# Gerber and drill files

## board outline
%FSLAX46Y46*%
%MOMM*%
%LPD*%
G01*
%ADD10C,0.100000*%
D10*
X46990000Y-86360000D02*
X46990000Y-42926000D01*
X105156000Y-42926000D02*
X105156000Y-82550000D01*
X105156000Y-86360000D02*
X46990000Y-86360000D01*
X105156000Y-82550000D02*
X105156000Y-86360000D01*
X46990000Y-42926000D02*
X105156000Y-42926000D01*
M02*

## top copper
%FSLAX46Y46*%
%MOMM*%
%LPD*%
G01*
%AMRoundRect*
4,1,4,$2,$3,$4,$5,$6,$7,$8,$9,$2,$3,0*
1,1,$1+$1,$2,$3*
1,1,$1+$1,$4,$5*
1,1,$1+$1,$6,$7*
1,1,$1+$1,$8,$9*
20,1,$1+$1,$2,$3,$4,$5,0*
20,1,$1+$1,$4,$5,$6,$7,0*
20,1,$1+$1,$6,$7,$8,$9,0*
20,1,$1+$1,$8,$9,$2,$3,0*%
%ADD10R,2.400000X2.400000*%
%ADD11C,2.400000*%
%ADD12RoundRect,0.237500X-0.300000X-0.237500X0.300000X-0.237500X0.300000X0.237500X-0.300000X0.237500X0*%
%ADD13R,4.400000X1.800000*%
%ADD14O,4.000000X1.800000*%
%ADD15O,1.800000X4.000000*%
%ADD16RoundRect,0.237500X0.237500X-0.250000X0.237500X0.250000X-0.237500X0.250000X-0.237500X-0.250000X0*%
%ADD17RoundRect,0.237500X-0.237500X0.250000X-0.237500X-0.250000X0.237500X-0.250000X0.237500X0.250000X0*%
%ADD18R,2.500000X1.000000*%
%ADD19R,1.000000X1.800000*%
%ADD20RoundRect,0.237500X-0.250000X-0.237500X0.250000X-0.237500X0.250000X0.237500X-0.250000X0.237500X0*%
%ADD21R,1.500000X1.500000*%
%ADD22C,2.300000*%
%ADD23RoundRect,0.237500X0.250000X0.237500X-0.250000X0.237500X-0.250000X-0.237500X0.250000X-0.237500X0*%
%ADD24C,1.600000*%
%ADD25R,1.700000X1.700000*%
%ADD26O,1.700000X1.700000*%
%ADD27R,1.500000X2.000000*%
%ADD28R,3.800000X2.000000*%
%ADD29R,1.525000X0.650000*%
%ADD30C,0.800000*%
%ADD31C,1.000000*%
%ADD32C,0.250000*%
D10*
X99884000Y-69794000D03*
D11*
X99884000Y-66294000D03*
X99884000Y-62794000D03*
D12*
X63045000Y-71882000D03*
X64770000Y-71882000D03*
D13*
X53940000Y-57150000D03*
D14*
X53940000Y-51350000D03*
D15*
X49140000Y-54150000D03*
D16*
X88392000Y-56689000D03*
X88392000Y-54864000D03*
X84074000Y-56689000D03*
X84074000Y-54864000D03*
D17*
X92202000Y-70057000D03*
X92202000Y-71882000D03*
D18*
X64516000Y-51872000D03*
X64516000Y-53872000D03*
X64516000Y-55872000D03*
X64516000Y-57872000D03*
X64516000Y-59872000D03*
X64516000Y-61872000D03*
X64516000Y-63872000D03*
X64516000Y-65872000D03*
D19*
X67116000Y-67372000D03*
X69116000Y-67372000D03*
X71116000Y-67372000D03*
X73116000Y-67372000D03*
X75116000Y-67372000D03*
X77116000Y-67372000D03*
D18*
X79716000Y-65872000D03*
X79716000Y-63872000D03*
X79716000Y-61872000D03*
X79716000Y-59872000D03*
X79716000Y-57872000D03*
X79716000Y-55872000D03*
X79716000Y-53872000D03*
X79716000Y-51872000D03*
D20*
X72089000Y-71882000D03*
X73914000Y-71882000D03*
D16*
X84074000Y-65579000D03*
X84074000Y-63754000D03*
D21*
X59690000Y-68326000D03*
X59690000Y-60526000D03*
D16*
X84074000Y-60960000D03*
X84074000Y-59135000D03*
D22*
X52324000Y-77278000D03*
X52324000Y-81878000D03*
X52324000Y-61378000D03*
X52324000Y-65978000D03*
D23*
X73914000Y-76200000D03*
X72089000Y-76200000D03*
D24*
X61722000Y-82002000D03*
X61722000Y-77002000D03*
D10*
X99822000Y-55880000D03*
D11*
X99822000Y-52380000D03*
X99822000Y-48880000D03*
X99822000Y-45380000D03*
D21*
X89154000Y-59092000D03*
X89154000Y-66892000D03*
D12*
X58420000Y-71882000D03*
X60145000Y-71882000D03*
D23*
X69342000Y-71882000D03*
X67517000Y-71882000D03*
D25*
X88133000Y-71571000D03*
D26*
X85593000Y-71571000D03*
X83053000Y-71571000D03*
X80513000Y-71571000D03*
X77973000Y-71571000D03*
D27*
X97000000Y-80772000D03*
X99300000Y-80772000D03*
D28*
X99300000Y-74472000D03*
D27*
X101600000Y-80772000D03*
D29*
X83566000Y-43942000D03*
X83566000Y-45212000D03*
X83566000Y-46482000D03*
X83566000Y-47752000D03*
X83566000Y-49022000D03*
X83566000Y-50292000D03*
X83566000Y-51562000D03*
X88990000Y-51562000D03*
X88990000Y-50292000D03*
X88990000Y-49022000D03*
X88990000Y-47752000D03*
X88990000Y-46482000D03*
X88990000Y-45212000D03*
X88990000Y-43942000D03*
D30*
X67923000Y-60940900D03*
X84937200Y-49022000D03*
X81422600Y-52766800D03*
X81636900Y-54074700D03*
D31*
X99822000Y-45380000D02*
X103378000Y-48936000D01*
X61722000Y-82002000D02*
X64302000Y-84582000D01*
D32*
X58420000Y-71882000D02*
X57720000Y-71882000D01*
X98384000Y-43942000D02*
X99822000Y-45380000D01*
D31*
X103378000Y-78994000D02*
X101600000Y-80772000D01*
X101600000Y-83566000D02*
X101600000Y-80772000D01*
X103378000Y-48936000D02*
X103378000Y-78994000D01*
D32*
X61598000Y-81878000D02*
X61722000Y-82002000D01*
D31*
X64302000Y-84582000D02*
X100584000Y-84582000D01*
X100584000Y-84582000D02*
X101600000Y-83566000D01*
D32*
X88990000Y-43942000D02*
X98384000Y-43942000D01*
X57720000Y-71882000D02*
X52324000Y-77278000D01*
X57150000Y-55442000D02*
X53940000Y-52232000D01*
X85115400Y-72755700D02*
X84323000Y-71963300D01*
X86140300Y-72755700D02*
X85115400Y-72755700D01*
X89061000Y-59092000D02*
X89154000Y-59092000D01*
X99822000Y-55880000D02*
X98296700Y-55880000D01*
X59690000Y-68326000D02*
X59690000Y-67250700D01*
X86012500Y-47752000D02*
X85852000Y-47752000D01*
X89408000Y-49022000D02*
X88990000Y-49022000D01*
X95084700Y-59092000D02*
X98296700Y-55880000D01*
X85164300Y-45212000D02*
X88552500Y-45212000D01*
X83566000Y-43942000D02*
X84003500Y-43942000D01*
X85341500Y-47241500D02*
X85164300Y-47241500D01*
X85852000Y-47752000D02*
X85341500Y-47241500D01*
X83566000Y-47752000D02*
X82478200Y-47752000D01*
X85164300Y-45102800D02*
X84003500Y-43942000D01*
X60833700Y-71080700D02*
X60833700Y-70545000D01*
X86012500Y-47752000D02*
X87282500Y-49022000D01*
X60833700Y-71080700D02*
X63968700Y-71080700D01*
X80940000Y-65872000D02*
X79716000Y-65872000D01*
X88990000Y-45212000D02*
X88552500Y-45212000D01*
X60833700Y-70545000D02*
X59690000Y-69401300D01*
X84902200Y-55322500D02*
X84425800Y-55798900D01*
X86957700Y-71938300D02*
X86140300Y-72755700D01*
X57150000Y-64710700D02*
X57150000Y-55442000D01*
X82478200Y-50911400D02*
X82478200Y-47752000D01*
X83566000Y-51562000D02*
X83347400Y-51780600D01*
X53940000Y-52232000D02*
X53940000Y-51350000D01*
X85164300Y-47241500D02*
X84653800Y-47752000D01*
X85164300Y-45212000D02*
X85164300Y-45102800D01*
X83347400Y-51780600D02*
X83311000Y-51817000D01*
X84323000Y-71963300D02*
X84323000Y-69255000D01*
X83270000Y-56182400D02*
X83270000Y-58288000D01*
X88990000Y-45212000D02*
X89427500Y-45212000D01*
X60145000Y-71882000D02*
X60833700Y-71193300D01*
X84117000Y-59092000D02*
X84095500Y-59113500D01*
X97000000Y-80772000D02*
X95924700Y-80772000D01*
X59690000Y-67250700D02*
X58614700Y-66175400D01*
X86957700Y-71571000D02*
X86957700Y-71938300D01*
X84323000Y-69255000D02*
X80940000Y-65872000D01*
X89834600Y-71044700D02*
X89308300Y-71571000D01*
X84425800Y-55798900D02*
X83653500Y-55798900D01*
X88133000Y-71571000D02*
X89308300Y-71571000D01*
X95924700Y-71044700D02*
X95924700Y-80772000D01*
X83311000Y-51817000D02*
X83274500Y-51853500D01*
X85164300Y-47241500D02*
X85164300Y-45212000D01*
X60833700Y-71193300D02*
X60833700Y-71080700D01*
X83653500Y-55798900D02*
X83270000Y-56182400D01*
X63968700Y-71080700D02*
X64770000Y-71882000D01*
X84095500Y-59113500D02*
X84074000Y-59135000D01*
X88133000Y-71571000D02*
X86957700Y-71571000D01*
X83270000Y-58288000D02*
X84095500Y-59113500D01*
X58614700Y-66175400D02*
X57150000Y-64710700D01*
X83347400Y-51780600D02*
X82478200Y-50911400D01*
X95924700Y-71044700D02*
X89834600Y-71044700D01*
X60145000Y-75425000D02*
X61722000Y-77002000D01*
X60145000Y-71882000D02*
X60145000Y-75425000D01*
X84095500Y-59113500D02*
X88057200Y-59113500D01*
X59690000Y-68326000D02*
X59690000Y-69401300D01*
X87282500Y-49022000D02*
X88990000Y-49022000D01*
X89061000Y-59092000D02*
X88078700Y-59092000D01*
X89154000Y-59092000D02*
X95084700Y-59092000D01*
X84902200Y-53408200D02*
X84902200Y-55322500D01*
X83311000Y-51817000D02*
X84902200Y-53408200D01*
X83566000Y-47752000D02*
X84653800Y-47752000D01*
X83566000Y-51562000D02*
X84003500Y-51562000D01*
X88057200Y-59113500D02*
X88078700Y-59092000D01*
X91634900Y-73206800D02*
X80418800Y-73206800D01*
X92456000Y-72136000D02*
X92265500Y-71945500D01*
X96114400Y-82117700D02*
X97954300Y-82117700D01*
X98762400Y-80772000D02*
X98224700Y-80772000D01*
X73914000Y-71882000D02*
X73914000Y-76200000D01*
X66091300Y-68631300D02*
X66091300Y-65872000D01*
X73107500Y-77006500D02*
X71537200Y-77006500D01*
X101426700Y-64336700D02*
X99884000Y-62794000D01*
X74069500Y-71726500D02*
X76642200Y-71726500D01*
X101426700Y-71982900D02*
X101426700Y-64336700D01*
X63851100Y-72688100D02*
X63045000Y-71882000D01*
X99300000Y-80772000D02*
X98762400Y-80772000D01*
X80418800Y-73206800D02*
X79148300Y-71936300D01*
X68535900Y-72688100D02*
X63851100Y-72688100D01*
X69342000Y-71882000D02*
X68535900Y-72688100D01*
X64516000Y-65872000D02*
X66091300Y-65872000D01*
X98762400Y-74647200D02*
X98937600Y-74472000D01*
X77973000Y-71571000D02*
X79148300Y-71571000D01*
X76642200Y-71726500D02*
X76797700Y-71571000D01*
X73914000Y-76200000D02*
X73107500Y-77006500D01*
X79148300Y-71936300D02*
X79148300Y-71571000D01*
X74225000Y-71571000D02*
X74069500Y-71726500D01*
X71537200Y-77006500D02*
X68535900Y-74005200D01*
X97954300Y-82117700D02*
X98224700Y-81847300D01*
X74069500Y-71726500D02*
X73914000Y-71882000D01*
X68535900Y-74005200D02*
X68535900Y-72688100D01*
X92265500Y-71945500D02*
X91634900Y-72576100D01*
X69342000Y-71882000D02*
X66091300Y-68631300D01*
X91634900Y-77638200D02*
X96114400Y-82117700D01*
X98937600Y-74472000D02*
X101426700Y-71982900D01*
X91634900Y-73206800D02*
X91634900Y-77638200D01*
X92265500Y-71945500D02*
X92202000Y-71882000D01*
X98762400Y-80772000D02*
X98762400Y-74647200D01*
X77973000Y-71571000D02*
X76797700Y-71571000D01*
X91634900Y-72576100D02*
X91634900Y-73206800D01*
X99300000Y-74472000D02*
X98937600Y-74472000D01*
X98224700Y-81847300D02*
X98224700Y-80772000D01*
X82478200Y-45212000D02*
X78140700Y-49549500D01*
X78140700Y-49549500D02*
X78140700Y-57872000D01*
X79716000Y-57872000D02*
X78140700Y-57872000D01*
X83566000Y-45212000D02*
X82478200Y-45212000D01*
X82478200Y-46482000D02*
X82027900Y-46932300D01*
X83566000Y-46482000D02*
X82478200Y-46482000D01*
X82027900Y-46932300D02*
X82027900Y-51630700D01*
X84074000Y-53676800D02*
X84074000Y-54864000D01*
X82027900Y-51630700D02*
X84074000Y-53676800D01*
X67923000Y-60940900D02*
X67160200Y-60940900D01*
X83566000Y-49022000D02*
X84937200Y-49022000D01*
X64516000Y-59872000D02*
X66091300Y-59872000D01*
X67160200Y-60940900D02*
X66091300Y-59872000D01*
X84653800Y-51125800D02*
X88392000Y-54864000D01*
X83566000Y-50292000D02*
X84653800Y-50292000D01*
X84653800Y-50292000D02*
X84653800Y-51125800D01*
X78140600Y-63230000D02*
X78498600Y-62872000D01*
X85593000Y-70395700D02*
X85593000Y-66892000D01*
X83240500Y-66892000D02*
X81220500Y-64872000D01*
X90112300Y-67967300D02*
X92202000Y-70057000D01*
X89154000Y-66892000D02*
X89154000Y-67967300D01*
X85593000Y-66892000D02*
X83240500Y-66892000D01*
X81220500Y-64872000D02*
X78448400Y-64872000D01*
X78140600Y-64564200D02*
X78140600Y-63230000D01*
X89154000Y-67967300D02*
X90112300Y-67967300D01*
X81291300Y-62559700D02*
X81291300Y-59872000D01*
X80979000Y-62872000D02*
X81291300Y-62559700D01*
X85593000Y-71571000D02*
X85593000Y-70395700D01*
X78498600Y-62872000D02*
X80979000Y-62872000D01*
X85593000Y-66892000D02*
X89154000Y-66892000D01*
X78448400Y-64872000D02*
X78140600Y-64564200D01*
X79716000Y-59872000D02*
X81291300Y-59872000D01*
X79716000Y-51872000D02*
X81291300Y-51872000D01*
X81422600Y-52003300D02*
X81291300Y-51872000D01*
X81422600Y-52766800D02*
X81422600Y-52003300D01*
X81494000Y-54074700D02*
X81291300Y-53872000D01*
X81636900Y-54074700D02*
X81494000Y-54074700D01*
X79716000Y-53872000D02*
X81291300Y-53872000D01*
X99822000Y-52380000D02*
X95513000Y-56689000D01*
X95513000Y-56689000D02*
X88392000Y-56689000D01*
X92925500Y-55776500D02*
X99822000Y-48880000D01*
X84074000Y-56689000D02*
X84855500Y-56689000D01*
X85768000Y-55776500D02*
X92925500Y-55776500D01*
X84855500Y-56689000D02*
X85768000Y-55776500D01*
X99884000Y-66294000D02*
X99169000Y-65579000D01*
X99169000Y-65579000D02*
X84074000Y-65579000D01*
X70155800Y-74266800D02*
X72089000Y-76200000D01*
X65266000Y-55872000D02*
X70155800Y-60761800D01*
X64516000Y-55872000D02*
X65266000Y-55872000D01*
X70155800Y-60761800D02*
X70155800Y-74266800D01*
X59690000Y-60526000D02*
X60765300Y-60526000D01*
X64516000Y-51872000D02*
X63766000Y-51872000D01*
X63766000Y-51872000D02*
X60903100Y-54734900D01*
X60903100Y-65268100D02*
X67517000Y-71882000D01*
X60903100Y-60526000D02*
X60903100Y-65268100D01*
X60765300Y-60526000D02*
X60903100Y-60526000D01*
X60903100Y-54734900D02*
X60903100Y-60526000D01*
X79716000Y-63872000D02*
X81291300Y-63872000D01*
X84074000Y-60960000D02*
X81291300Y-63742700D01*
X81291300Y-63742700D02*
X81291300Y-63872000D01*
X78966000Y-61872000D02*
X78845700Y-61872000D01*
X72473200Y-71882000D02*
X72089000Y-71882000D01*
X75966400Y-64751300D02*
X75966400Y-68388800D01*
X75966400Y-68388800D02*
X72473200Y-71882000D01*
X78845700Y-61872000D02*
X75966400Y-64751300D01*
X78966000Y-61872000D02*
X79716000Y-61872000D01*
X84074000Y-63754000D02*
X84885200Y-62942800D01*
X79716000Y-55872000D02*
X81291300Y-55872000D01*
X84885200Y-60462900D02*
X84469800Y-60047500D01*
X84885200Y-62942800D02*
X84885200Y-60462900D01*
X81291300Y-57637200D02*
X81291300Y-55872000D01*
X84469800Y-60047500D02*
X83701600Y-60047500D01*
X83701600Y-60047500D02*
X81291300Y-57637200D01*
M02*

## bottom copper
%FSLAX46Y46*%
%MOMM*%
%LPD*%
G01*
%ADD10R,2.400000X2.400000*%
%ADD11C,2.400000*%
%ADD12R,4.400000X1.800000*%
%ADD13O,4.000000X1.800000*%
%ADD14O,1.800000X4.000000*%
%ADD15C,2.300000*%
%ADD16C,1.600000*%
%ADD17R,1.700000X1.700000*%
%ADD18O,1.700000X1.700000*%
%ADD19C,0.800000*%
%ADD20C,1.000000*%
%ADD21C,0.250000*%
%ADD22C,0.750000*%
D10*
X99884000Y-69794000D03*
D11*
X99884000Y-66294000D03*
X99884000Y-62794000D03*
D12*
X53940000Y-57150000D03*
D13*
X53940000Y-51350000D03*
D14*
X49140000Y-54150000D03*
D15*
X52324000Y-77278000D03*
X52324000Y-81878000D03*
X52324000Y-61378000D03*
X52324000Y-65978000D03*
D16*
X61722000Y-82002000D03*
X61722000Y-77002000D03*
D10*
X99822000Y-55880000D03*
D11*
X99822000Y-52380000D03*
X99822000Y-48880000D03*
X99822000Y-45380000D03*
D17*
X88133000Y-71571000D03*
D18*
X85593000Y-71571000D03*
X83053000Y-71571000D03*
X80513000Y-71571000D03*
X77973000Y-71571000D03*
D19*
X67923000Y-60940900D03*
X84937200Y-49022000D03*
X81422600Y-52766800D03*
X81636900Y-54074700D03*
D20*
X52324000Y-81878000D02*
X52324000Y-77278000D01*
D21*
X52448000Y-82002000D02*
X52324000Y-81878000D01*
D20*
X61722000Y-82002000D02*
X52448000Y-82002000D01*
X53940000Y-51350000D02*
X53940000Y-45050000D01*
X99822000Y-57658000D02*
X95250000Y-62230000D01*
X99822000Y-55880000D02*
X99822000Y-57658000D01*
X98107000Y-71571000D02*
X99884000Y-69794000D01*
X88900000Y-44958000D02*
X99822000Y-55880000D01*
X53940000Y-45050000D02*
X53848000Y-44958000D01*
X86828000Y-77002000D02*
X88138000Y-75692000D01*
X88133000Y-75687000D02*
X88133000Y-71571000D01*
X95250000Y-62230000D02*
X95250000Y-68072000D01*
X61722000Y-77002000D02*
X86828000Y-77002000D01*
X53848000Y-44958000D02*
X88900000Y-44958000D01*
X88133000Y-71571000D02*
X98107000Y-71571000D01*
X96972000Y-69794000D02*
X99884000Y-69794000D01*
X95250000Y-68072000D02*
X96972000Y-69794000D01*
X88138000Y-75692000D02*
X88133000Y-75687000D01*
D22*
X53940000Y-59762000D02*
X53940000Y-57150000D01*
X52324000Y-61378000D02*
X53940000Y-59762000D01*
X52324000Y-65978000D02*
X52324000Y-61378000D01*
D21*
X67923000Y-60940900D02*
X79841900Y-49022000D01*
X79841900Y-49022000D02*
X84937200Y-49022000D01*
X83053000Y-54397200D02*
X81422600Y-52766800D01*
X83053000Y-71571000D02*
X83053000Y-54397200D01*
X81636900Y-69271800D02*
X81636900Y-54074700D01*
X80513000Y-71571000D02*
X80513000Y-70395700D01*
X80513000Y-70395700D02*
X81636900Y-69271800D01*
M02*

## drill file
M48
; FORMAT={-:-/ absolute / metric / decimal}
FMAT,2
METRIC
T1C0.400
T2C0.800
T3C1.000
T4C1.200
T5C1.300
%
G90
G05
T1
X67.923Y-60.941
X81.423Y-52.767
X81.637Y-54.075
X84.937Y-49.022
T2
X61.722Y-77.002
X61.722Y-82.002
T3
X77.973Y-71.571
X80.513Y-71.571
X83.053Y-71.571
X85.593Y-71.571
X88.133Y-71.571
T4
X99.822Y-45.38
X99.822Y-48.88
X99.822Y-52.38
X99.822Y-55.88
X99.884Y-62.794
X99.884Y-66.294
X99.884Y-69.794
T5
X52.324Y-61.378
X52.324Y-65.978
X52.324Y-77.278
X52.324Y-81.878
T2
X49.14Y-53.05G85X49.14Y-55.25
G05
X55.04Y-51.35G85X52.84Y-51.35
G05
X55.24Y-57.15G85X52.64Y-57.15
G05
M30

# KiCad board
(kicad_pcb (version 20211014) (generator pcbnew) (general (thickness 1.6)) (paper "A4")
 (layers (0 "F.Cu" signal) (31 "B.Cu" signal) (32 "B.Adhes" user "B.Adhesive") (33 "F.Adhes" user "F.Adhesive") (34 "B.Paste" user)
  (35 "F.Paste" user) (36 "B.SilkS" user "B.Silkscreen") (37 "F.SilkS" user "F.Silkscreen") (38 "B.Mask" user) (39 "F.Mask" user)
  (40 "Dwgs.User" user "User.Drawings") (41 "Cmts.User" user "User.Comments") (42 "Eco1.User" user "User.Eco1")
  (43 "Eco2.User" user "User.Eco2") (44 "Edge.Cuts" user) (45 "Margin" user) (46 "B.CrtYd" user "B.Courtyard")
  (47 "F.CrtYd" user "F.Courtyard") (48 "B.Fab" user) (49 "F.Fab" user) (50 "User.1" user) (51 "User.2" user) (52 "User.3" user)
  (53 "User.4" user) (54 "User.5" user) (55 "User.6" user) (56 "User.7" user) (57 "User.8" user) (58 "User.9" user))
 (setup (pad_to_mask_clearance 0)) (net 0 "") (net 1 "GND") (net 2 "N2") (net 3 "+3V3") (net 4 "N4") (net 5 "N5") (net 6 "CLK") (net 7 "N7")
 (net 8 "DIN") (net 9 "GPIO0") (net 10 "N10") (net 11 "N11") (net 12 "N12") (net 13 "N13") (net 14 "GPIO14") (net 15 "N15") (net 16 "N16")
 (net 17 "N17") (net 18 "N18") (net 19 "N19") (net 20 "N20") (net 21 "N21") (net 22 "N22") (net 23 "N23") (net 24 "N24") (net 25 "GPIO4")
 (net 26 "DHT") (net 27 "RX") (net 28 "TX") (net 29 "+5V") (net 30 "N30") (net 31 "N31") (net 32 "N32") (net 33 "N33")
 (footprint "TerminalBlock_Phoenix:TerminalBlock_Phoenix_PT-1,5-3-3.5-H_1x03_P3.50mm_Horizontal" (layer "F.Cu") (at 99.884 69.794 90)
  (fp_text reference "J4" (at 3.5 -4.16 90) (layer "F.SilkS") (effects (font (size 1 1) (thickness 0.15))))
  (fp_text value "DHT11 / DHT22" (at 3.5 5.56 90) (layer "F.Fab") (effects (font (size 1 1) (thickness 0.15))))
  (pad "1" thru_hole rect locked (at 0 0 90) (size 2.4 2.4) (drill 1.2) (layers *.Cu *.Mask) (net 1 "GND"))
  (pad "2" thru_hole circle locked (at 3.5 0 90) (size 2.4 2.4) (drill 1.2) (layers *.Cu *.Mask) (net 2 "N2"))
  (pad "3" thru_hole circle locked (at 7 0 90) (size 2.4 2.4) (drill 1.2) (layers *.Cu *.Mask) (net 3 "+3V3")))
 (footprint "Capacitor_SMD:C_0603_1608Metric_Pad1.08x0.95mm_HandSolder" (layer "F.Cu") (at 63.9075 71.882)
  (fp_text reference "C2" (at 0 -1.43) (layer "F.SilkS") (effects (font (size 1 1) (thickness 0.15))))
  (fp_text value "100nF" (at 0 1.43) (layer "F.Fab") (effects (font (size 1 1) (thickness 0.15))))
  (pad "1" smd roundrect locked (at -0.8625 0) (size 1.075 0.95) (layers "F.Cu" "F.Paste" "F.Mask") (roundrect_rratio 0.25) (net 3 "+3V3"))
  (pad "2" smd roundrect locked (at 0.8625 0) (size 1.075 0.95) (layers "F.Cu" "F.Paste" "F.Mask") (roundrect_rratio 0.25) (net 1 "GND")))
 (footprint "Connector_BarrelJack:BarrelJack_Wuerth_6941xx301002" (layer "F.Cu") (at 53.94 57.15 180)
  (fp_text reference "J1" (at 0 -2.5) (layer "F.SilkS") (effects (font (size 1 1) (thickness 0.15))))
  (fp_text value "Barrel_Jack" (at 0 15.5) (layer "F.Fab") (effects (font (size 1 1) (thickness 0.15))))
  (pad "1" thru_hole rect locked (at 0 0 180) (size 4.4 1.8) (drill oval 3.4 0.8) (layers *.Cu *.Mask) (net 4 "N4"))
  (pad "2" thru_hole oval locked (at 0 5.8 180) (size 4 1.8) (drill oval 3 0.8) (layers *.Cu *.Mask) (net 1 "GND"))
  (pad "3" thru_hole oval locked (at 4.8 3 270) (size 4 1.8) (drill oval 3 0.8) (layers *.Cu *.Mask)))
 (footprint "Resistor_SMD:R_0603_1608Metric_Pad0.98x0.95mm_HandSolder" (layer "F.Cu") (at 88.392 55.7765 90)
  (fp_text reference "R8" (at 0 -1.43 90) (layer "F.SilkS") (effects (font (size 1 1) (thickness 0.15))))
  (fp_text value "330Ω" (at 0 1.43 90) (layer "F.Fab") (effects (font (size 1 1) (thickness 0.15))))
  (pad "1" smd roundrect locked (at -0.9125 0 90) (size 0.975 0.95) (layers "F.Cu" "F.Paste" "F.Mask") (roundrect_rratio 0.25) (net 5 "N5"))
  (pad "2" smd roundrect locked (at 0.9125 0 90) (size 0.975 0.95) (layers "F.Cu" "F.Paste" "F.Mask") (roundrect_rratio 0.25) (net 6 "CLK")))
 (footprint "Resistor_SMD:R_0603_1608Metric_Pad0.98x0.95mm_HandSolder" (layer "F.Cu") (at 84.074 55.7765 90)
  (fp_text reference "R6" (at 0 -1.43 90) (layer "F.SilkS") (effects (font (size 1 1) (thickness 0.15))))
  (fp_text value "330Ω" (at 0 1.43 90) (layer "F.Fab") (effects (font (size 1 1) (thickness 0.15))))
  (pad "1" smd roundrect locked (at -0.9125 0 90) (size 0.975 0.95) (layers "F.Cu" "F.Paste" "F.Mask") (roundrect_rratio 0.25) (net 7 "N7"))
  (pad "2" smd roundrect locked (at 0.9125 0 90) (size 0.975 0.95) (layers "F.Cu" "F.Paste" "F.Mask") (roundrect_rratio 0.25) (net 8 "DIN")))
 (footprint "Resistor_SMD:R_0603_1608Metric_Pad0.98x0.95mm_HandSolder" (layer "F.Cu") (at 92.202 70.9695 -90)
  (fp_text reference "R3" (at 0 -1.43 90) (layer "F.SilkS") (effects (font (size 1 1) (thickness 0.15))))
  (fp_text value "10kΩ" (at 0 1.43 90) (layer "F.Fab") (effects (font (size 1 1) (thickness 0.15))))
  (pad "1" smd roundrect locked (at -0.9125 0 270) (size 0.975 0.95) (layers "F.Cu" "F.Paste" "F.Mask") (roundrect_rratio 0.25)
   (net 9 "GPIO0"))
  (pad "2" smd roundrect locked (at 0.9125 0 270) (size 0.975 0.95) (layers "F.Cu" "F.Paste" "F.Mask") (roundrect_rratio 0.25)
   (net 3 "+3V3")))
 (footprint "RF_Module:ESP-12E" (layer "F.Cu") (at 72.116 55.372)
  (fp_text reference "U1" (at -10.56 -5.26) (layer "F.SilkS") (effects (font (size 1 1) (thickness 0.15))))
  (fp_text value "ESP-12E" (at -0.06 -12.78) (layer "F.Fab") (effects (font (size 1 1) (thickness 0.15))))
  (pad "1" smd rect locked (at -7.6 -3.5) (size 2.5 1) (layers "F.Cu" "F.Paste" "F.Mask") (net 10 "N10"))
  (pad "2" smd rect locked (at -7.6 -1.5) (size 2.5 1) (layers "F.Cu" "F.Paste" "F.Mask") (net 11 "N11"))
  (pad "3" smd rect locked (at -7.6 0.5) (size 2.5 1) (layers "F.Cu" "F.Paste" "F.Mask") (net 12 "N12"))
  (pad "4" smd rect locked (at -7.6 2.5) (size 2.5 1) (layers "F.Cu" "F.Paste" "F.Mask") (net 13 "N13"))
  (pad "5" smd rect locked (at -7.6 4.5) (size 2.5 1) (layers "F.Cu" "F.Paste" "F.Mask") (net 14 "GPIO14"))
  (pad "6" smd rect locked (at -7.6 6.5) (size 2.5 1) (layers "F.Cu" "F.Paste" "F.Mask") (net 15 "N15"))
  (pad "7" smd rect locked (at -7.6 8.5) (size 2.5 1) (layers "F.Cu" "F.Paste" "F.Mask") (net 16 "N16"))
  (pad "8" smd rect locked (at -7.6 10.5) (size 2.5 1) (layers "F.Cu" "F.Paste" "F.Mask") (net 3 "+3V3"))
  (pad "9" smd rect locked (at -5 12) (size 1 1.8) (layers "F.Cu" "F.Paste" "F.Mask") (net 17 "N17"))
  (pad "10" smd rect locked (at -3 12) (size 1 1.8) (layers "F.Cu" "F.Paste" "F.Mask") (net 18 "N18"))
  (pad "11" smd rect locked (at -1 12) (size 1 1.8) (layers "F.Cu" "F.Paste" "F.Mask") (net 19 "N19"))
  (pad "12" smd rect locked (at 1 12) (size 1 1.8) (layers "F.Cu" "F.Paste" "F.Mask") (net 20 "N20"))
  (pad "13" smd rect locked (at 3 12) (size 1 1.8) (layers "F.Cu" "F.Paste" "F.Mask") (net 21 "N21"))
  (pad "14" smd rect locked (at 5 12) (size 1 1.8) (layers "F.Cu" "F.Paste" "F.Mask") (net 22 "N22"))
  (pad "15" smd rect locked (at 7.6 10.5) (size 2.5 1) (layers "F.Cu" "F.Paste" "F.Mask") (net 1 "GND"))
  (pad "16" smd rect locked (at 7.6 8.5) (size 2.5 1) (layers "F.Cu" "F.Paste" "F.Mask") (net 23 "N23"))
  (pad "17" smd rect locked (at 7.6 6.5) (size 2.5 1) (layers "F.Cu" "F.Paste" "F.Mask") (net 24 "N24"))
  (pad "18" smd rect locked (at 7.6 4.5) (size 2.5 1) (layers "F.Cu" "F.Paste" "F.Mask") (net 9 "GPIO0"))
  (pad "19" smd rect locked (at 7.6 2.5) (size 2.5 1) (layers "F.Cu" "F.Paste" "F.Mask") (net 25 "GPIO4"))
  (pad "20" smd rect locked (at 7.6 0.5) (size 2.5 1) (layers "F.Cu" "F.Paste" "F.Mask") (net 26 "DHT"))
  (pad "21" smd rect locked (at 7.6 -1.5) (size 2.5 1) (layers "F.Cu" "F.Paste" "F.Mask") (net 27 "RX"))
  (pad "22" smd rect locked (at 7.6 -3.5) (size 2.5 1) (layers "F.Cu" "F.Paste" "F.Mask") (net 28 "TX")))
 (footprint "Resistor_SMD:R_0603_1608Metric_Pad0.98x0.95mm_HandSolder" (layer "F.Cu") (at 73.0015 71.882)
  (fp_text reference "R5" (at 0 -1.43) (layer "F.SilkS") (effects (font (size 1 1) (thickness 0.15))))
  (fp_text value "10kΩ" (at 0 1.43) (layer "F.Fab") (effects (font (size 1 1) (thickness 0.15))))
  (pad "1" smd roundrect locked (at -0.9125 0) (size 0.975 0.95) (layers "F.Cu" "F.Paste" "F.Mask") (roundrect_rratio 0.25) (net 24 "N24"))
  (pad "2" smd roundrect locked (at 0.9125 0) (size 0.975 0.95) (layers "F.Cu" "F.Paste" "F.Mask") (roundrect_rratio 0.25) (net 3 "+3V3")))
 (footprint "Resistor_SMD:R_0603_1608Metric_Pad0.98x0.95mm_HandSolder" (layer "F.Cu") (at 84.074 64.6665 90)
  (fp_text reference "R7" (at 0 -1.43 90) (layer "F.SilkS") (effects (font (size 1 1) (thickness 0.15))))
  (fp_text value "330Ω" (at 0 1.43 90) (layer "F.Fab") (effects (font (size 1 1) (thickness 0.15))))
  (pad "1" smd roundrect locked (at -0.9125 0 90) (size 0.975 0.95) (layers "F.Cu" "F.Paste" "F.Mask") (roundrect_rratio 0.25) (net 2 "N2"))
  (pad "2" smd roundrect locked (at 0.9125 0 90) (size 0.975 0.95) (layers "F.Cu" "F.Paste" "F.Mask") (roundrect_rratio 0.25) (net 26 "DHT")))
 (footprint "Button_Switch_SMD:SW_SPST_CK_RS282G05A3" (layer "F.Cu") (at 59.69 64.426 90)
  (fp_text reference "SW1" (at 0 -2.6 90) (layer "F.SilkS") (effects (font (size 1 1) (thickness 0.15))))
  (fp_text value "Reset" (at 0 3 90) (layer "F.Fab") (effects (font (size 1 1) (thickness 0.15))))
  (pad "1" smd rect locked (at -3.9 0 90) (size 1.5 1.5) (layers "F.Cu" "F.Paste" "F.Mask") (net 1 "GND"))
  (pad "2" smd rect locked (at 3.9 0 90) (size 1.5 1.5) (layers "F.Cu" "F.Paste" "F.Mask") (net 10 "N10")))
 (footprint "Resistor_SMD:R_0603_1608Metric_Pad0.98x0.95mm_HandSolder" (layer "F.Cu") (at 84.074 60.0475 90)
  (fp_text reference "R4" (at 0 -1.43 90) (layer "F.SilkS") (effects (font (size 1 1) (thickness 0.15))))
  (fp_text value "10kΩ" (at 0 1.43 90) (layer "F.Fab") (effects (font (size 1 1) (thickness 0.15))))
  (pad "1" smd roundrect locked (at -0.9125 0 90) (size 0.975 0.95) (layers "F.Cu" "F.Paste" "F.Mask") (roundrect_rratio 0.25)
   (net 23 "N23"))
  (pad "2" smd roundrect locked (at 0.9125 0 90) (size 0.975 0.95) (layers "F.Cu" "F.Paste" "F.Mask") (roundrect_rratio 0.25) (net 1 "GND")))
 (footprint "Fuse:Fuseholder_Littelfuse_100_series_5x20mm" (layer "F.Cu") (at 52.324 81.878 90)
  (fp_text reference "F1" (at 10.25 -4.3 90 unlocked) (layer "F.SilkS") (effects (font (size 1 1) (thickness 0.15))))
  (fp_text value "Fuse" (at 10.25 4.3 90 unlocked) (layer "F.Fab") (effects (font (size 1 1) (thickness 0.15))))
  (pad "1" thru_hole circle (at 4.6 0 90) (size 2.3 2.3) (drill 1.3) (layers *.Cu *.Mask) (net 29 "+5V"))
  (pad "1" thru_hole circle (at 0 0 90) (size 2.3 2.3) (drill 1.3) (layers *.Cu *.Mask) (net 29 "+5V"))
  (pad "2" thru_hole circle (at 20.5 0 90) (size 2.3 2.3) (drill 1.3) (layers *.Cu *.Mask) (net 4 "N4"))
  (pad "2" thru_hole circle (at 15.9 0 90) (size 2.3 2.3) (drill 1.3) (layers *.Cu *.Mask) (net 4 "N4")))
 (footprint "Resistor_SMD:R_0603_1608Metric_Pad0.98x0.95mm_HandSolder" (layer "F.Cu") (at 73.0015 76.2 180)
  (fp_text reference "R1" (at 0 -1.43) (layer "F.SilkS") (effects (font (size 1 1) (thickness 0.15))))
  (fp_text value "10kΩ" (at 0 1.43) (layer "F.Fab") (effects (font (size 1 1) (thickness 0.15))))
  (pad "1" smd roundrect locked (at -0.9125 0 180) (size 0.975 0.95) (layers "F.Cu" "F.Paste" "F.Mask") (roundrect_rratio 0.25)
   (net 3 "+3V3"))
  (pad "2" smd roundrect locked (at 0.9125 0 180) (size 0.975 0.95) (layers "F.Cu" "F.Paste" "F.Mask") (roundrect_rratio 0.25)
   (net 12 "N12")))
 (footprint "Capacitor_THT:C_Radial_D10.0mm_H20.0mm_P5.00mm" (layer "F.Cu") (at 61.722 82.002 90)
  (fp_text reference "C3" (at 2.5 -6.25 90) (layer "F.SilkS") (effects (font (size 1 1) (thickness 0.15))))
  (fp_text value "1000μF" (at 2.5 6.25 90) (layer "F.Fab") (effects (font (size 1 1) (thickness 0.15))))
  (pad "1" thru_hole circle locked (at 0 0 90) (size 1.6 1.6) (drill 0.8) (layers *.Cu *.Mask) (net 29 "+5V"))
  (pad "2" thru_hole circle locked (at 5 0 90) (size 1.6 1.6) (drill 0.8) (layers *.Cu *.Mask) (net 1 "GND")))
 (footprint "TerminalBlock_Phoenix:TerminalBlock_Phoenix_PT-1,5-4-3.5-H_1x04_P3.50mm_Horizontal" (layer "F.Cu") (at 99.822 55.88 90)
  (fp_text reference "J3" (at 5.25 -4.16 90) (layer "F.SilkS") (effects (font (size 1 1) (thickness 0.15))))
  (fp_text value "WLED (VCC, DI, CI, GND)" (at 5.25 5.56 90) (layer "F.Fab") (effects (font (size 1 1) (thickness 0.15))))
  (pad "1" thru_hole rect locked (at 0 0 90) (size 2.4 2.4) (drill 1.2) (layers *.Cu *.Mask) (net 1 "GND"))
  (pad "2" thru_hole circle locked (at 3.5 0 90) (size 2.4 2.4) (drill 1.2) (layers *.Cu *.Mask) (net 5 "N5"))
  (pad "3" thru_hole circle locked (at 7 0 90) (size 2.4 2.4) (drill 1.2) (layers *.Cu *.Mask) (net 7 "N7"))
  (pad "4" thru_hole circle locked (at 10.5 0 90) (size 2.4 2.4) (drill 1.2) (layers *.Cu *.Mask) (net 29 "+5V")))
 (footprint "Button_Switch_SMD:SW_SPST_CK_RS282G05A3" (layer "F.Cu") (at 89.154 62.992 -90)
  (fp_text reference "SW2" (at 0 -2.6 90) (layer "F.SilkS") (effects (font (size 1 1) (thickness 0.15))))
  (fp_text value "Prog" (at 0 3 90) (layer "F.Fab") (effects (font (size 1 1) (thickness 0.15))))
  (pad "1" smd rect locked (at -3.9 0 270) (size 1.5 1.5) (layers "F.Cu" "F.Paste" "F.Mask") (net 1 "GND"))
  (pad "2" smd rect locked (at 3.9 0 270) (size 1.5 1.5) (layers "F.Cu" "F.Paste" "F.Mask") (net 9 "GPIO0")))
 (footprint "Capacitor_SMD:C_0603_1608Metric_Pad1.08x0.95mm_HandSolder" (layer "F.Cu") (at 59.2825 71.882)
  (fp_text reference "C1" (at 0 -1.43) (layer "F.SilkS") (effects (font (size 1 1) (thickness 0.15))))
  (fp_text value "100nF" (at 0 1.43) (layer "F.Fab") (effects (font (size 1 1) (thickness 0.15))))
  (pad "1" smd roundrect locked (at -0.8625 0) (size 1.075 0.95) (layers "F.Cu" "F.Paste" "F.Mask") (roundrect_rratio 0.25) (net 29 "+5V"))
  (pad "2" smd roundrect locked (at 0.8625 0) (size 1.075 0.95) (layers "F.Cu" "F.Paste" "F.Mask") (roundrect_rratio 0.25) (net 1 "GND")))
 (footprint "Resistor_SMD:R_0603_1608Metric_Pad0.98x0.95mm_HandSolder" (layer "F.Cu") (at 68.4295 71.882 180)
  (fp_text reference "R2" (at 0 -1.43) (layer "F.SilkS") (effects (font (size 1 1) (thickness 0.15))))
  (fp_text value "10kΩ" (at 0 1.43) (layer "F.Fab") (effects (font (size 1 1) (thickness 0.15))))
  (pad "1" smd roundrect locked (at -0.9125 0 180) (size 0.975 0.95) (layers "F.Cu" "F.Paste" "F.Mask") (roundrect_rratio 0.25)
   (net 3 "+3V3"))
  (pad "2" smd roundrect locked (at 0.9125 0 180) (size 0.975 0.95) (layers "F.Cu" "F.Paste" "F.Mask") (roundrect_rratio 0.25)
   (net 10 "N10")))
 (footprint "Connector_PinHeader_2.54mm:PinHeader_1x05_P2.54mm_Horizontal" (layer "F.Cu") (at 88.133 71.571 -90)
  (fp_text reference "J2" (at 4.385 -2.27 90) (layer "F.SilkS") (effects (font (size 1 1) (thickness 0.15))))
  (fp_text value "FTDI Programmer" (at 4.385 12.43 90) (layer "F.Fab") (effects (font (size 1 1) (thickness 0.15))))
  (pad "1" thru_hole rect locked (at 0 0 270) (size 1.7 1.7) (drill 1) (layers *.Cu *.Mask) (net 1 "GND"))
  (pad "2" thru_hole oval locked (at 0 2.54 270) (size 1.7 1.7) (drill 1) (layers *.Cu *.Mask) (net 9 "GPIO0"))
  (pad "3" thru_hole oval locked (at 0 5.08 270) (size 1.7 1.7) (drill 1) (layers *.Cu *.Mask) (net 28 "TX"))
  (pad "4" thru_hole oval locked (at 0 7.62 270) (size 1.7 1.7) (drill 1) (layers *.Cu *.Mask) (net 27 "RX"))
  (pad "5" thru_hole oval locked (at 0 10.16 270) (size 1.7 1.7) (drill 1) (layers *.Cu *.Mask) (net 3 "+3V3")))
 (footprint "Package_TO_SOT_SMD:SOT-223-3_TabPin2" (layer "F.Cu") (at 99.3 77.622 90)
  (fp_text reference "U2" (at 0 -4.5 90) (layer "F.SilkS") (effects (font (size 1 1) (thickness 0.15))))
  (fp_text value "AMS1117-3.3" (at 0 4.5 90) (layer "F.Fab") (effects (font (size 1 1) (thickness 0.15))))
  (pad "1" smd rect locked (at -3.15 -2.3 90) (size 2 1.5) (layers "F.Cu" "F.Paste" "F.Mask") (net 1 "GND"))
  (pad "2" smd rect locked (at -3.15 0 90) (size 2 1.5) (layers "F.Cu" "F.Paste" "F.Mask") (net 3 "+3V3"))
  (pad "2" smd rect locked (at 3.15 0 90) (size 2 3.8) (layers "F.Cu" "F.Paste" "F.Mask") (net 3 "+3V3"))
  (pad "3" smd rect locked (at -3.15 2.3 90) (size 2 1.5) (layers "F.Cu" "F.Paste" "F.Mask") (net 29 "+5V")))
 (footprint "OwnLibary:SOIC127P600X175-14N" (layer "F.Cu") (at 86.278 47.752)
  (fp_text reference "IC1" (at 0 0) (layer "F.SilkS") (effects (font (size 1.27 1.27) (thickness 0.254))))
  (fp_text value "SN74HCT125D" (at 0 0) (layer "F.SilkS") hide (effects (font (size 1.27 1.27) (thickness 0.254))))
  (pad "1" smd rect locked (at -2.712 -3.81 90) (size 0.65 1.525) (layers "F.Cu" "F.Paste" "F.Mask") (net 1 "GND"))
  (pad "2" smd rect locked (at -2.712 -2.54 90) (size 0.65 1.525) (layers "F.Cu" "F.Paste" "F.Mask") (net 25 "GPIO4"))
  (pad "3" smd rect locked (at -2.712 -1.27 90) (size 0.65 1.525) (layers "F.Cu" "F.Paste" "F.Mask") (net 8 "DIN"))
  (pad "4" smd rect locked (at -2.712 0 90) (size 0.65 1.525) (layers "F.Cu" "F.Paste" "F.Mask") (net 1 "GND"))
  (pad "5" smd rect locked (at -2.712 1.27 90) (size 0.65 1.525) (layers "F.Cu" "F.Paste" "F.Mask") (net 14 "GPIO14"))
  (pad "6" smd rect locked (at -2.712 2.54 90) (size 0.65 1.525) (layers "F.Cu" "F.Paste" "F.Mask") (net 6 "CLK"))
  (pad "7" smd rect locked (at -2.712 3.81 90) (size 0.65 1.525) (layers "F.Cu" "F.Paste" "F.Mask") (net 1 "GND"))
  (pad "8" smd rect locked (at 2.712 3.81 90) (size 0.65 1.525) (layers "F.Cu" "F.Paste" "F.Mask") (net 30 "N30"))
  (pad "9" smd rect locked (at 2.712 2.54 90) (size 0.65 1.525) (layers "F.Cu" "F.Paste" "F.Mask") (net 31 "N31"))
  (pad "10" smd rect locked (at 2.712 1.27 90) (size 0.65 1.525) (layers "F.Cu" "F.Paste" "F.Mask") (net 1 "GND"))
  (pad "11" smd rect locked (at 2.712 0 90) (size 0.65 1.525) (layers "F.Cu" "F.Paste" "F.Mask") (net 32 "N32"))
  (pad "12" smd rect locked (at 2.712 -1.27 90) (size 0.65 1.525) (layers "F.Cu" "F.Paste" "F.Mask") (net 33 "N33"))
  (pad "13" smd rect locked (at 2.712 -2.54 90) (size 0.65 1.525) (layers "F.Cu" "F.Paste" "F.Mask") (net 1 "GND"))
  (pad "14" smd rect locked (at 2.712 -3.81 90) (size 0.65 1.525) (layers "F.Cu" "F.Paste" "F.Mask") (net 29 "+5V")))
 (gr_line (start 46.99 86.36) (end 46.99 42.926) (layer "Edge.Cuts") (width 0.1))
 (gr_line (start 105.156 42.926) (end 105.156 82.55) (layer "Edge.Cuts") (width 0.1))
 (gr_line (start 105.156 86.36) (end 46.99 86.36) (layer "Edge.Cuts") (width 0.1))
 (gr_line (start 105.156 82.55) (end 105.156 86.36) (layer "Edge.Cuts") (width 0.1))
 (gr_line (start 46.99 42.926) (end 105.156 42.926) (layer "Edge.Cuts") (width 0.1))
 (segment (start 99.822 45.38) (end 103.378 48.936) (width 1) (layer "F.Cu") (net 29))
 (segment (start 61.722 82.002) (end 64.302 84.582) (width 1) (layer "F.Cu") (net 29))
 (segment (start 58.42 71.882) (end 57.72 71.882) (width 0.25) (layer "F.Cu") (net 29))
 (segment (start 98.384 43.942) (end 99.822 45.38) (width 0.25) (layer "F.Cu") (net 29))
 (segment (start 103.378 78.994) (end 101.6 80.772) (width 1) (layer "F.Cu") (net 29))
 (segment (start 101.6 83.566) (end 101.6 80.772) (width 1) (layer "F.Cu") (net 29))
 (segment (start 103.378 48.936) (end 103.378 78.994) (width 1) (layer "F.Cu") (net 29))
 (segment (start 61.598 81.878) (end 61.722 82.002) (width 0.25) (layer "F.Cu") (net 29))
 (segment (start 64.302 84.582) (end 100.584 84.582) (width 1) (layer "F.Cu") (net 29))
 (segment (start 100.584 84.582) (end 101.6 83.566) (width 1) (layer "F.Cu") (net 29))
 (segment (start 88.99 43.942) (end 98.384 43.942) (width 0.25) (layer "F.Cu") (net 29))
 (segment (start 57.72 71.882) (end 52.324 77.278) (width 0.25) (layer "F.Cu") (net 29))
 (segment (start 52.324 81.878) (end 52.324 77.278) (width 1) (layer "B.Cu") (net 29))
 (segment (start 52.448 82.002) (end 52.324 81.878) (width 0.25) (layer "B.Cu") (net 29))
 (segment (start 61.722 82.002) (end 52.448 82.002) (width 1) (layer "B.Cu") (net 29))
 (segment (start 57.15 55.442) (end 53.94 52.232) (width 0.25) (layer "F.Cu") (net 1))
 (segment (start 85.1154 72.7557) (end 84.323 71.9633) (width 0.25) (layer "F.Cu") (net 1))
 (segment (start 86.1403 72.7557) (end 85.1154 72.7557) (width 0.25) (layer "F.Cu") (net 1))
 (segment (start 89.061 59.092) (end 89.154 59.092) (width 0.25) (layer "F.Cu") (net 1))
 (segment (start 99.822 55.88) (end 98.2967 55.88) (width 0.25) (layer "F.Cu") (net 1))
 (segment (start 59.69 68.326) (end 59.69 67.2507) (width 0.25) (layer "F.Cu") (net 1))
 (segment (start 86.0125 47.752) (end 85.852 47.752) (width 0.25) (layer "F.Cu") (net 1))
 (segment (start 89.408 49.022) (end 88.99 49.022) (width 0.25) (layer "F.Cu") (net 1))
 (segment (start 95.0847 59.092) (end 98.2967 55.88) (width 0.25) (layer "F.Cu") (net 1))
 (segment (start 85.1643 45.212) (end 88.5525 45.212) (width 0.25) (layer "F.Cu") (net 1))
 (segment (start 83.566 43.942) (end 84.0035 43.942) (width 0.25) (layer "F.Cu") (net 1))
 (segment (start 85.3415 47.2415) (end 85.1643 47.2415) (width 0.25) (layer "F.Cu") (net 1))
 (segment (start 85.852 47.752) (end 85.3415 47.2415) (width 0.25) (layer "F.Cu") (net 1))
 (segment (start 83.566 47.752) (end 82.4782 47.752) (width 0.25) (layer "F.Cu") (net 1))
 (segment (start 85.1643 45.1028) (end 84.0035 43.942) (width 0.25) (layer "F.Cu") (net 1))
 (segment (start 60.8337 71.0807) (end 60.8337 70.545) (width 0.25) (layer "F.Cu") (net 1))
 (segment (start 86.0125 47.752) (end 87.2825 49.022) (width 0.25) (layer "F.Cu") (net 1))
 (segment (start 60.8337 71.0807) (end 63.9687 71.0807) (width 0.25) (layer "F.Cu") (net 1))
 (segment (start 80.94 65.872) (end 79.716 65.872) (width 0.25) (layer "F.Cu") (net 1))
 (segment (start 88.99 45.212) (end 88.5525 45.212) (width 0.25) (layer "F.Cu") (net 1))
 (segment (start 60.8337 70.545) (end 59.69 69.4013) (width 0.25) (layer "F.Cu") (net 1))
 (segment (start 84.9022 55.3225) (end 84.4258 55.7989) (width 0.25) (layer "F.Cu") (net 1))
 (segment (start 86.9577 71.9383) (end 86.1403 72.7557) (width 0.25) (layer "F.Cu") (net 1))
 (segment (start 57.15 64.7107) (end 57.15 55.442) (width 0.25) (layer "F.Cu") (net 1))
 (segment (start 82.4782 50.9114) (end 82.4782 47.752) (width 0.25) (layer "F.Cu") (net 1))
 (segment (start 83.566 51.562) (end 83.3474 51.7806) (width 0.25) (layer "F.Cu") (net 1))
 (segment (start 53.94 52.232) (end 53.94 51.35) (width 0.25) (layer "F.Cu") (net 1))
 (segment (start 85.1643 47.2415) (end 84.6538 47.752) (width 0.25) (layer "F.Cu") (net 1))
 (segment (start 85.1643 45.212) (end 85.1643 45.1028) (width 0.25) (layer "F.Cu") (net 1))
 (segment (start 83.3474 51.7806) (end 83.311 51.817) (width 0.25) (layer "F.Cu") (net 1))
 (segment (start 84.323 71.9633) (end 84.323 69.255) (width 0.25) (layer "F.Cu") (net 1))
 (segment (start 83.27 56.1824) (end 83.27 58.288) (width 0.25) (layer "F.Cu") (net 1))
 (segment (start 88.99 45.212) (end 89.4275 45.212) (width 0.25) (layer "F.Cu") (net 1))
 (segment (start 60.145 71.882) (end 60.8337 71.1933) (width 0.25) (layer "F.Cu") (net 1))
 (segment (start 84.117 59.092) (end 84.0955 59.1135) (width 0.25) (layer "F.Cu") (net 1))
 (segment (start 97 80.772) (end 95.9247 80.772) (width 0.25) (layer "F.Cu") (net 1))
 (segment (start 59.69 67.2507) (end 58.6147 66.1754) (width 0.25) (layer "F.Cu") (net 1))
 (segment (start 86.9577 71.571) (end 86.9577 71.9383) (width 0.25) (layer "F.Cu") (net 1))
 (segment (start 84.323 69.255) (end 80.94 65.872) (width 0.25) (layer "F.Cu") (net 1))
 (segment (start 89.8346 71.0447) (end 89.3083 71.571) (width 0.25) (layer "F.Cu") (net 1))
 (segment (start 84.4258 55.7989) (end 83.6535 55.7989) (width 0.25) (layer "F.Cu") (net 1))
 (segment (start 88.133 71.571) (end 89.3083 71.571) (width 0.25) (layer "F.Cu") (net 1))
 (segment (start 95.9247 71.0447) (end 95.9247 80.772) (width 0.25) (layer "F.Cu") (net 1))
 (segment (start 83.311 51.817) (end 83.2745 51.8535) (width 0.25) (layer "F.Cu") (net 1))
 (segment (start 85.1643 47.2415) (end 85.1643 45.212) (width 0.25) (layer "F.Cu") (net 1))
 (segment (start 60.8337 71.1933) (end 60.8337 71.0807) (width 0.25) (layer "F.Cu") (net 1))
 (segment (start 83.6535 55.7989) (end 83.27 56.1824) (width 0.25) (layer "F.Cu") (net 1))
 (segment (start 63.9687 71.0807) (end 64.77 71.882) (width 0.25) (layer "F.Cu") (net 1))
 (segment (start 84.0955 59.1135) (end 84.074 59.135) (width 0.25) (layer "F.Cu") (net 1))
 (segment (start 88.133 71.571) (end 86.9577 71.571) (width 0.25) (layer "F.Cu") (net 1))
 (segment (start 83.27 58.288) (end 84.0955 59.1135) (width 0.25) (layer "F.Cu") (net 1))
 (segment (start 58.6147 66.1754) (end 57.15 64.7107) (width 0.25) (layer "F.Cu") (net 1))
 (segment (start 83.3474 51.7806) (end 82.4782 50.9114) (width 0.25) (layer "F.Cu") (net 1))
 (segment (start 95.9247 71.0447) (end 89.8346 71.0447) (width 0.25) (layer "F.Cu") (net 1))
 (segment (start 60.145 75.425) (end 61.722 77.002) (width 0.25) (layer "F.Cu") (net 1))
 (segment (start 60.145 71.882) (end 60.145 75.425) (width 0.25) (layer "F.Cu") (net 1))
 (segment (start 84.0955 59.1135) (end 88.0572 59.1135) (width 0.25) (layer "F.Cu") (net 1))
 (segment (start 59.69 68.326) (end 59.69 69.4013) (width 0.25) (layer "F.Cu") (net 1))
 (segment (start 87.2825 49.022) (end 88.99 49.022) (width 0.25) (layer "F.Cu") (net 1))
 (segment (start 89.061 59.092) (end 88.0787 59.092) (width 0.25) (layer "F.Cu") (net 1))
 (segment (start 89.154 59.092) (end 95.0847 59.092) (width 0.25) (layer "F.Cu") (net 1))
 (segment (start 84.9022 53.4082) (end 84.9022 55.3225) (width 0.25) (layer "F.Cu") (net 1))
 (segment (start 83.311 51.817) (end 84.9022 53.4082) (width 0.25) (layer "F.Cu") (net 1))
 (segment (start 83.566 47.752) (end 84.6538 47.752) (width 0.25) (layer "F.Cu") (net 1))
 (segment (start 83.566 51.562) (end 84.0035 51.562) (width 0.25) (layer "F.Cu") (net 1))
 (segment (start 88.0572 59.1135) (end 88.0787 59.092) (width 0.25) (layer "F.Cu") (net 1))
 (segment (start 53.94 51.35) (end 53.94 45.05) (width 1) (layer "B.Cu") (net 1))
 (segment (start 99.822 57.658) (end 95.25 62.23) (width 1) (layer "B.Cu") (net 1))
 (segment (start 99.822 55.88) (end 99.822 57.658) (width 1) (layer "B.Cu") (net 1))
 (segment (start 98.107 71.571) (end 99.884 69.794) (width 1) (layer "B.Cu") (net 1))
 (segment (start 88.9 44.958) (end 99.822 55.88) (width 1) (layer "B.Cu") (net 1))
 (segment (start 53.94 45.05) (end 53.848 44.958) (width 1) (layer "B.Cu") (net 1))
 (segment (start 86.828 77.002) (end 88.138 75.692) (width 1) (layer "B.Cu") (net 1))
 (segment (start 88.133 75.687) (end 88.133 71.571) (width 1) (layer "B.Cu") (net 1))
 (segment (start 95.25 62.23) (end 95.25 68.072) (width 1) (layer "B.Cu") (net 1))
 (segment (start 61.722 77.002) (end 86.828 77.002) (width 1) (layer "B.Cu") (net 1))
 (segment (start 53.848 44.958) (end 88.9 44.958) (width 1) (layer "B.Cu") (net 1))
 (segment (start 88.133 71.571) (end 98.107 71.571) (width 1) (layer "B.Cu") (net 1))
 (segment (start 96.972 69.794) (end 99.884 69.794) (width 1) (layer "B.Cu") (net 1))
 (segment (start 95.25 68.072) (end 96.972 69.794) (width 1) (layer "B.Cu") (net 1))
 (segment (start 88.138 75.692) (end 88.133 75.687) (width 1) (layer "B.Cu") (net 1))
 (segment (start 91.6349 73.2068) (end 80.4188 73.2068) (width 0.25) (layer "F.Cu") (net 3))
 (segment (start 92.456 72.136) (end 92.2655 71.9455) (width 0.25) (layer "F.Cu") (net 3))
 (segment (start 96.1144 82.1177) (end 97.9543 82.1177) (width 0.25) (layer "F.Cu") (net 3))
 (segment (start 98.7624 80.772) (end 98.2247 80.772) (width 0.25) (layer "F.Cu") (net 3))
 (segment (start 73.914 71.882) (end 73.914 76.2) (width 0.25) (layer "F.Cu") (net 3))
 (segment (start 66.0913 68.6313) (end 66.0913 65.872) (width 0.25) (layer "F.Cu") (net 3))
 (segment (start 73.1075 77.0065) (end 71.5372 77.0065) (width 0.25) (layer "F.Cu") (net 3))
 (segment (start 101.4267 64.3367) (end 99.884 62.794) (width 0.25) (layer "F.Cu") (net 3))
 (segment (start 74.0695 71.7265) (end 76.6422 71.7265) (width 0.25) (layer "F.Cu") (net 3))
 (segment (start 101.4267 71.9829) (end 101.4267 64.3367) (width 0.25) (layer "F.Cu") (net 3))
 (segment (start 63.8511 72.6881) (end 63.045 71.882) (width 0.25) (layer "F.Cu") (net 3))
 (segment (start 99.3 80.772) (end 98.7624 80.772) (width 0.25) (layer "F.Cu") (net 3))
 (segment (start 80.4188 73.2068) (end 79.1483 71.9363) (width 0.25) (layer "F.Cu") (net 3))
 (segment (start 68.5359 72.6881) (end 63.8511 72.6881) (width 0.25) (layer "F.Cu") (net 3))
 (segment (start 69.342 71.882) (end 68.5359 72.6881) (width 0.25) (layer "F.Cu") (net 3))
 (segment (start 64.516 65.872) (end 66.0913 65.872) (width 0.25) (layer "F.Cu") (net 3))
 (segment (start 98.7624 74.6472) (end 98.9376 74.472) (width 0.25) (layer "F.Cu") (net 3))
 (segment (start 77.973 71.571) (end 79.1483 71.571) (width 0.25) (layer "F.Cu") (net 3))
 (segment (start 76.6422 71.7265) (end 76.7977 71.571) (width 0.25) (layer "F.Cu") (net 3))
 (segment (start 73.914 76.2) (end 73.1075 77.0065) (width 0.25) (layer "F.Cu") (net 3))
 (segment (start 79.1483 71.9363) (end 79.1483 71.571) (width 0.25) (layer "F.Cu") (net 3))
 (segment (start 74.225 71.571) (end 74.0695 71.7265) (width 0.25) (layer "F.Cu") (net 3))
 (segment (start 71.5372 77.0065) (end 68.5359 74.0052) (width 0.25) (layer "F.Cu") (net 3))
 (segment (start 97.9543 82.1177) (end 98.2247 81.8473) (width 0.25) (layer "F.Cu") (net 3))
 (segment (start 74.0695 71.7265) (end 73.914 71.882) (width 0.25) (layer "F.Cu") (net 3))
 (segment (start 68.5359 74.0052) (end 68.5359 72.6881) (width 0.25) (layer "F.Cu") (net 3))
 (segment (start 92.2655 71.9455) (end 91.6349 72.5761) (width 0.25) (layer "F.Cu") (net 3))
 (segment (start 69.342 71.882) (end 66.0913 68.6313) (width 0.25) (layer "F.Cu") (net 3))
 (segment (start 91.6349 77.6382) (end 96.1144 82.1177) (width 0.25) (layer "F.Cu") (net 3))
 (segment (start 98.9376 74.472) (end 101.4267 71.9829) (width 0.25) (layer "F.Cu") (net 3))
 (segment (start 91.6349 73.2068) (end 91.6349 77.6382) (width 0.25) (layer "F.Cu") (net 3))
 (segment (start 92.2655 71.9455) (end 92.202 71.882) (width 0.25) (layer "F.Cu") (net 3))
 (segment (start 98.7624 80.772) (end 98.7624 74.6472) (width 0.25) (layer "F.Cu") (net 3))
 (segment (start 77.973 71.571) (end 76.7977 71.571) (width 0.25) (layer "F.Cu") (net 3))
 (segment (start 91.6349 72.5761) (end 91.6349 73.2068) (width 0.25) (layer "F.Cu") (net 3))
 (segment (start 99.3 74.472) (end 98.9376 74.472) (width 0.25) (layer "F.Cu") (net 3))
 (segment (start 98.2247 81.8473) (end 98.2247 80.772) (width 0.25) (layer "F.Cu") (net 3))
 (segment (start 53.94 59.762) (end 53.94 57.15) (width 0.75) (layer "B.Cu") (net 4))
 (segment (start 52.324 61.378) (end 53.94 59.762) (width 0.75) (layer "B.Cu") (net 4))
 (segment (start 52.324 65.978) (end 52.324 61.378) (width 0.75) (layer "B.Cu") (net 4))
 (segment (start 82.4782 45.212) (end 78.1407 49.5495) (width 0.25) (layer "F.Cu") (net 25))
 (segment (start 78.1407 49.5495) (end 78.1407 57.872) (width 0.25) (layer "F.Cu") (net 25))
 (segment (start 79.716 57.872) (end 78.1407 57.872) (width 0.25) (layer "F.Cu") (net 25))
 (segment (start 83.566 45.212) (end 82.4782 45.212) (width 0.25) (layer "F.Cu") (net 25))
 (segment (start 82.4782 46.482) (end 82.0279 46.9323) (width 0.25) (layer "F.Cu") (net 8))
 (segment (start 83.566 46.482) (end 82.4782 46.482) (width 0.25) (layer "F.Cu") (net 8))
 (segment (start 82.0279 46.9323) (end 82.0279 51.6307) (width 0.25) (layer "F.Cu") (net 8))
 (segment (start 84.074 53.6768) (end 84.074 54.864) (width 0.25) (layer "F.Cu") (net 8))
 (segment (start 82.0279 51.6307) (end 84.074 53.6768) (width 0.25) (layer "F.Cu") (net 8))
 (segment (start 67.923 60.9409) (end 67.1602 60.9409) (width 0.25) (layer "F.Cu") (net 14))
 (segment (start 83.566 49.022) (end 84.9372 49.022) (width 0.25) (layer "F.Cu") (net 14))
 (segment (start 64.516 59.872) (end 66.0913 59.872) (width 0.25) (layer "F.Cu") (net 14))
 (segment (start 67.1602 60.9409) (end 66.0913 59.872) (width 0.25) (layer "F.Cu") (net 14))
 (via (at 67.923 60.9409) (size 0.8) (drill 0.4) (layers "F.Cu" "B.Cu") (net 14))
 (via (at 84.9372 49.022) (size 0.8) (drill 0.4) (layers "F.Cu" "B.Cu") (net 14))
 (segment (start 67.923 60.9409) (end 79.8419 49.022) (width 0.25) (layer "B.Cu") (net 14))
 (segment (start 79.8419 49.022) (end 84.9372 49.022) (width 0.25) (layer "B.Cu") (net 14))
 (segment (start 84.6538 51.1258) (end 88.392 54.864) (width 0.25) (layer "F.Cu") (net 6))
 (segment (start 83.566 50.292) (end 84.6538 50.292) (width 0.25) (layer "F.Cu") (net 6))
 (segment (start 84.6538 50.292) (end 84.6538 51.1258) (width 0.25) (layer "F.Cu") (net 6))
 (segment (start 78.1406 63.23) (end 78.4986 62.872) (width 0.25) (layer "F.Cu") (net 9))
 (segment (start 85.593 70.3957) (end 85.593 66.892) (width 0.25) (layer "F.Cu") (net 9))
 (segment (start 83.2405 66.892) (end 81.2205 64.872) (width 0.25) (layer "F.Cu") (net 9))
 (segment (start 90.1123 67.9673) (end 92.202 70.057) (width 0.25) (layer "F.Cu") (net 9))
 (segment (start 89.154 66.892) (end 89.154 67.9673) (width 0.25) (layer "F.Cu") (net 9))
 (segment (start 85.593 66.892) (end 83.2405 66.892) (width 0.25) (layer "F.Cu") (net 9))
 (segment (start 81.2205 64.872) (end 78.4484 64.872) (width 0.25) (layer "F.Cu") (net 9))
 (segment (start 78.1406 64.5642) (end 78.1406 63.23) (width 0.25) (layer "F.Cu") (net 9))
 (segment (start 89.154 67.9673) (end 90.1123 67.9673) (width 0.25) (layer "F.Cu") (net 9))
 (segment (start 81.2913 62.5597) (end 81.2913 59.872) (width 0.25) (layer "F.Cu") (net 9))
 (segment (start 80.979 62.872) (end 81.2913 62.5597) (width 0.25) (layer "F.Cu") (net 9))
 (segment (start 85.593 71.571) (end 85.593 70.3957) (width 0.25) (layer "F.Cu") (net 9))
 (segment (start 78.4986 62.872) (end 80.979 62.872) (width 0.25) (layer "F.Cu") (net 9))
 (segment (start 85.593 66.892) (end 89.154 66.892) (width 0.25) (layer "F.Cu") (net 9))
 (segment (start 78.4484 64.872) (end 78.1406 64.5642) (width 0.25) (layer "F.Cu") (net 9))
 (segment (start 79.716 59.872) (end 81.2913 59.872) (width 0.25) (layer "F.Cu") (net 9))
 (segment (start 79.716 51.872) (end 81.2913 51.872) (width 0.25) (layer "F.Cu") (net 28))
 (segment (start 81.4226 52.0033) (end 81.2913 51.872) (width 0.25) (layer "F.Cu") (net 28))
 (segment (start 81.4226 52.7668) (end 81.4226 52.0033) (width 0.25) (layer "F.Cu") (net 28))
 (via (at 81.4226 52.7668) (size 0.8) (drill 0.4) (layers "F.Cu" "B.Cu") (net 28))
 (segment (start 83.053 54.3972) (end 81.4226 52.7668) (width 0.25) (layer "B.Cu") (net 28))
 (segment (start 83.053 71.571) (end 83.053 54.3972) (width 0.25) (layer "B.Cu") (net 28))
 (segment (start 81.494 54.0747) (end 81.2913 53.872) (width 0.25) (layer "F.Cu") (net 27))
 (segment (start 81.6369 54.0747) (end 81.494 54.0747) (width 0.25) (layer "F.Cu") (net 27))
 (segment (start 79.716 53.872) (end 81.2913 53.872) (width 0.25) (layer "F.Cu") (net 27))
 (via (at 81.6369 54.0747) (size 0.8) (drill 0.4) (layers "F.Cu" "B.Cu") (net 27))
 (segment (start 81.6369 69.2718) (end 81.6369 54.0747) (width 0.25) (layer "B.Cu") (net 27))
 (segment (start 80.513 71.571) (end 80.513 70.3957) (width 0.25) (layer "B.Cu") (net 27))
 (segment (start 80.513 70.3957) (end 81.6369 69.2718) (width 0.25) (layer "B.Cu") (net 27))
 (segment (start 99.822 52.38) (end 95.513 56.689) (width 0.25) (layer "F.Cu") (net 5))
 (segment (start 95.513 56.689) (end 88.392 56.689) (width 0.25) (layer "F.Cu") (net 5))
 (segment (start 92.9255 55.7765) (end 99.822 48.88) (width 0.25) (layer "F.Cu") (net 7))
 (segment (start 84.074 56.689) (end 84.8555 56.689) (width 0.25) (layer "F.Cu") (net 7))
 (segment (start 85.768 55.7765) (end 92.9255 55.7765) (width 0.25) (layer "F.Cu") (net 7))
 (segment (start 84.8555 56.689) (end 85.768 55.7765) (width 0.25) (layer "F.Cu") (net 7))
 (segment (start 99.884 66.294) (end 99.169 65.579) (width 0.25) (layer "F.Cu") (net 2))
 (segment (start 99.169 65.579) (end 84.074 65.579) (width 0.25) (layer "F.Cu") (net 2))
 (segment (start 70.1558 74.2668) (end 72.089 76.2) (width 0.25) (layer "F.Cu") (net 12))
 (segment (start 65.266 55.872) (end 70.1558 60.7618) (width 0.25) (layer "F.Cu") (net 12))
 (segment (start 64.516 55.872) (end 65.266 55.872) (width 0.25) (layer "F.Cu") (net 12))
 (segment (start 70.1558 60.7618) (end 70.1558 74.2668) (width 0.25) (layer "F.Cu") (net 12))
 (segment (start 59.69 60.526) (end 60.7653 60.526) (width 0.25) (layer "F.Cu") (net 10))
 (segment (start 64.516 51.872) (end 63.766 51.872) (width 0.25) (layer "F.Cu") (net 10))
 (segment (start 63.766 51.872) (end 60.9031 54.7349) (width 0.25) (layer "F.Cu") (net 10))
 (segment (start 60.9031 65.2681) (end 67.517 71.882) (width 0.25) (layer "F.Cu") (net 10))
 (segment (start 60.9031 60.526) (end 60.9031 65.2681) (width 0.25) (layer "F.Cu") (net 10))
 (segment (start 60.7653 60.526) (end 60.9031 60.526) (width 0.25) (layer "F.Cu") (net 10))
 (segment (start 60.9031 54.7349) (end 60.9031 60.526) (width 0.25) (layer "F.Cu") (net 10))
 (segment (start 79.716 63.872) (end 81.2913 63.872) (width 0.25) (layer "F.Cu") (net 23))
 (segment (start 84.074 60.96) (end 81.2913 63.7427) (width 0.25) (layer "F.Cu") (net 23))
 (segment (start 81.2913 63.7427) (end 81.2913 63.872) (width 0.25) (layer "F.Cu") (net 23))
 (segment (start 78.966 61.872) (end 78.8457 61.872) (width 0.25) (layer "F.Cu") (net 24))
 (segment (start 72.4732 71.882) (end 72.089 71.882) (width 0.25) (layer "F.Cu") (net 24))
 (segment (start 75.9664 64.7513) (end 75.9664 68.3888) (width 0.25) (layer "F.Cu") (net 24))
 (segment (start 75.9664 68.3888) (end 72.4732 71.882) (width 0.25) (layer "F.Cu") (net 24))
 (segment (start 78.8457 61.872) (end 75.9664 64.7513) (width 0.25) (layer "F.Cu") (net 24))
 (segment (start 78.966 61.872) (end 79.716 61.872) (width 0.25) (layer "F.Cu") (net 24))
 (segment (start 84.074 63.754) (end 84.8852 62.9428) (width 0.25) (layer "F.Cu") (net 26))
 (segment (start 79.716 55.872) (end 81.2913 55.872) (width 0.25) (layer "F.Cu") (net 26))
 (segment (start 84.8852 60.4629) (end 84.4698 60.0475) (width 0.25) (layer "F.Cu") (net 26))
 (segment (start 84.8852 62.9428) (end 84.8852 60.4629) (width 0.25) (layer "F.Cu") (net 26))
 (segment (start 81.2913 57.6372) (end 81.2913 55.872) (width 0.25) (layer "F.Cu") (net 26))
 (segment (start 84.4698 60.0475) (end 83.7016 60.0475) (width 0.25) (layer "F.Cu") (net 26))
 (segment (start 83.7016 60.0475) (end 81.2913 57.6372) (width 0.25) (layer "F.Cu") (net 26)))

